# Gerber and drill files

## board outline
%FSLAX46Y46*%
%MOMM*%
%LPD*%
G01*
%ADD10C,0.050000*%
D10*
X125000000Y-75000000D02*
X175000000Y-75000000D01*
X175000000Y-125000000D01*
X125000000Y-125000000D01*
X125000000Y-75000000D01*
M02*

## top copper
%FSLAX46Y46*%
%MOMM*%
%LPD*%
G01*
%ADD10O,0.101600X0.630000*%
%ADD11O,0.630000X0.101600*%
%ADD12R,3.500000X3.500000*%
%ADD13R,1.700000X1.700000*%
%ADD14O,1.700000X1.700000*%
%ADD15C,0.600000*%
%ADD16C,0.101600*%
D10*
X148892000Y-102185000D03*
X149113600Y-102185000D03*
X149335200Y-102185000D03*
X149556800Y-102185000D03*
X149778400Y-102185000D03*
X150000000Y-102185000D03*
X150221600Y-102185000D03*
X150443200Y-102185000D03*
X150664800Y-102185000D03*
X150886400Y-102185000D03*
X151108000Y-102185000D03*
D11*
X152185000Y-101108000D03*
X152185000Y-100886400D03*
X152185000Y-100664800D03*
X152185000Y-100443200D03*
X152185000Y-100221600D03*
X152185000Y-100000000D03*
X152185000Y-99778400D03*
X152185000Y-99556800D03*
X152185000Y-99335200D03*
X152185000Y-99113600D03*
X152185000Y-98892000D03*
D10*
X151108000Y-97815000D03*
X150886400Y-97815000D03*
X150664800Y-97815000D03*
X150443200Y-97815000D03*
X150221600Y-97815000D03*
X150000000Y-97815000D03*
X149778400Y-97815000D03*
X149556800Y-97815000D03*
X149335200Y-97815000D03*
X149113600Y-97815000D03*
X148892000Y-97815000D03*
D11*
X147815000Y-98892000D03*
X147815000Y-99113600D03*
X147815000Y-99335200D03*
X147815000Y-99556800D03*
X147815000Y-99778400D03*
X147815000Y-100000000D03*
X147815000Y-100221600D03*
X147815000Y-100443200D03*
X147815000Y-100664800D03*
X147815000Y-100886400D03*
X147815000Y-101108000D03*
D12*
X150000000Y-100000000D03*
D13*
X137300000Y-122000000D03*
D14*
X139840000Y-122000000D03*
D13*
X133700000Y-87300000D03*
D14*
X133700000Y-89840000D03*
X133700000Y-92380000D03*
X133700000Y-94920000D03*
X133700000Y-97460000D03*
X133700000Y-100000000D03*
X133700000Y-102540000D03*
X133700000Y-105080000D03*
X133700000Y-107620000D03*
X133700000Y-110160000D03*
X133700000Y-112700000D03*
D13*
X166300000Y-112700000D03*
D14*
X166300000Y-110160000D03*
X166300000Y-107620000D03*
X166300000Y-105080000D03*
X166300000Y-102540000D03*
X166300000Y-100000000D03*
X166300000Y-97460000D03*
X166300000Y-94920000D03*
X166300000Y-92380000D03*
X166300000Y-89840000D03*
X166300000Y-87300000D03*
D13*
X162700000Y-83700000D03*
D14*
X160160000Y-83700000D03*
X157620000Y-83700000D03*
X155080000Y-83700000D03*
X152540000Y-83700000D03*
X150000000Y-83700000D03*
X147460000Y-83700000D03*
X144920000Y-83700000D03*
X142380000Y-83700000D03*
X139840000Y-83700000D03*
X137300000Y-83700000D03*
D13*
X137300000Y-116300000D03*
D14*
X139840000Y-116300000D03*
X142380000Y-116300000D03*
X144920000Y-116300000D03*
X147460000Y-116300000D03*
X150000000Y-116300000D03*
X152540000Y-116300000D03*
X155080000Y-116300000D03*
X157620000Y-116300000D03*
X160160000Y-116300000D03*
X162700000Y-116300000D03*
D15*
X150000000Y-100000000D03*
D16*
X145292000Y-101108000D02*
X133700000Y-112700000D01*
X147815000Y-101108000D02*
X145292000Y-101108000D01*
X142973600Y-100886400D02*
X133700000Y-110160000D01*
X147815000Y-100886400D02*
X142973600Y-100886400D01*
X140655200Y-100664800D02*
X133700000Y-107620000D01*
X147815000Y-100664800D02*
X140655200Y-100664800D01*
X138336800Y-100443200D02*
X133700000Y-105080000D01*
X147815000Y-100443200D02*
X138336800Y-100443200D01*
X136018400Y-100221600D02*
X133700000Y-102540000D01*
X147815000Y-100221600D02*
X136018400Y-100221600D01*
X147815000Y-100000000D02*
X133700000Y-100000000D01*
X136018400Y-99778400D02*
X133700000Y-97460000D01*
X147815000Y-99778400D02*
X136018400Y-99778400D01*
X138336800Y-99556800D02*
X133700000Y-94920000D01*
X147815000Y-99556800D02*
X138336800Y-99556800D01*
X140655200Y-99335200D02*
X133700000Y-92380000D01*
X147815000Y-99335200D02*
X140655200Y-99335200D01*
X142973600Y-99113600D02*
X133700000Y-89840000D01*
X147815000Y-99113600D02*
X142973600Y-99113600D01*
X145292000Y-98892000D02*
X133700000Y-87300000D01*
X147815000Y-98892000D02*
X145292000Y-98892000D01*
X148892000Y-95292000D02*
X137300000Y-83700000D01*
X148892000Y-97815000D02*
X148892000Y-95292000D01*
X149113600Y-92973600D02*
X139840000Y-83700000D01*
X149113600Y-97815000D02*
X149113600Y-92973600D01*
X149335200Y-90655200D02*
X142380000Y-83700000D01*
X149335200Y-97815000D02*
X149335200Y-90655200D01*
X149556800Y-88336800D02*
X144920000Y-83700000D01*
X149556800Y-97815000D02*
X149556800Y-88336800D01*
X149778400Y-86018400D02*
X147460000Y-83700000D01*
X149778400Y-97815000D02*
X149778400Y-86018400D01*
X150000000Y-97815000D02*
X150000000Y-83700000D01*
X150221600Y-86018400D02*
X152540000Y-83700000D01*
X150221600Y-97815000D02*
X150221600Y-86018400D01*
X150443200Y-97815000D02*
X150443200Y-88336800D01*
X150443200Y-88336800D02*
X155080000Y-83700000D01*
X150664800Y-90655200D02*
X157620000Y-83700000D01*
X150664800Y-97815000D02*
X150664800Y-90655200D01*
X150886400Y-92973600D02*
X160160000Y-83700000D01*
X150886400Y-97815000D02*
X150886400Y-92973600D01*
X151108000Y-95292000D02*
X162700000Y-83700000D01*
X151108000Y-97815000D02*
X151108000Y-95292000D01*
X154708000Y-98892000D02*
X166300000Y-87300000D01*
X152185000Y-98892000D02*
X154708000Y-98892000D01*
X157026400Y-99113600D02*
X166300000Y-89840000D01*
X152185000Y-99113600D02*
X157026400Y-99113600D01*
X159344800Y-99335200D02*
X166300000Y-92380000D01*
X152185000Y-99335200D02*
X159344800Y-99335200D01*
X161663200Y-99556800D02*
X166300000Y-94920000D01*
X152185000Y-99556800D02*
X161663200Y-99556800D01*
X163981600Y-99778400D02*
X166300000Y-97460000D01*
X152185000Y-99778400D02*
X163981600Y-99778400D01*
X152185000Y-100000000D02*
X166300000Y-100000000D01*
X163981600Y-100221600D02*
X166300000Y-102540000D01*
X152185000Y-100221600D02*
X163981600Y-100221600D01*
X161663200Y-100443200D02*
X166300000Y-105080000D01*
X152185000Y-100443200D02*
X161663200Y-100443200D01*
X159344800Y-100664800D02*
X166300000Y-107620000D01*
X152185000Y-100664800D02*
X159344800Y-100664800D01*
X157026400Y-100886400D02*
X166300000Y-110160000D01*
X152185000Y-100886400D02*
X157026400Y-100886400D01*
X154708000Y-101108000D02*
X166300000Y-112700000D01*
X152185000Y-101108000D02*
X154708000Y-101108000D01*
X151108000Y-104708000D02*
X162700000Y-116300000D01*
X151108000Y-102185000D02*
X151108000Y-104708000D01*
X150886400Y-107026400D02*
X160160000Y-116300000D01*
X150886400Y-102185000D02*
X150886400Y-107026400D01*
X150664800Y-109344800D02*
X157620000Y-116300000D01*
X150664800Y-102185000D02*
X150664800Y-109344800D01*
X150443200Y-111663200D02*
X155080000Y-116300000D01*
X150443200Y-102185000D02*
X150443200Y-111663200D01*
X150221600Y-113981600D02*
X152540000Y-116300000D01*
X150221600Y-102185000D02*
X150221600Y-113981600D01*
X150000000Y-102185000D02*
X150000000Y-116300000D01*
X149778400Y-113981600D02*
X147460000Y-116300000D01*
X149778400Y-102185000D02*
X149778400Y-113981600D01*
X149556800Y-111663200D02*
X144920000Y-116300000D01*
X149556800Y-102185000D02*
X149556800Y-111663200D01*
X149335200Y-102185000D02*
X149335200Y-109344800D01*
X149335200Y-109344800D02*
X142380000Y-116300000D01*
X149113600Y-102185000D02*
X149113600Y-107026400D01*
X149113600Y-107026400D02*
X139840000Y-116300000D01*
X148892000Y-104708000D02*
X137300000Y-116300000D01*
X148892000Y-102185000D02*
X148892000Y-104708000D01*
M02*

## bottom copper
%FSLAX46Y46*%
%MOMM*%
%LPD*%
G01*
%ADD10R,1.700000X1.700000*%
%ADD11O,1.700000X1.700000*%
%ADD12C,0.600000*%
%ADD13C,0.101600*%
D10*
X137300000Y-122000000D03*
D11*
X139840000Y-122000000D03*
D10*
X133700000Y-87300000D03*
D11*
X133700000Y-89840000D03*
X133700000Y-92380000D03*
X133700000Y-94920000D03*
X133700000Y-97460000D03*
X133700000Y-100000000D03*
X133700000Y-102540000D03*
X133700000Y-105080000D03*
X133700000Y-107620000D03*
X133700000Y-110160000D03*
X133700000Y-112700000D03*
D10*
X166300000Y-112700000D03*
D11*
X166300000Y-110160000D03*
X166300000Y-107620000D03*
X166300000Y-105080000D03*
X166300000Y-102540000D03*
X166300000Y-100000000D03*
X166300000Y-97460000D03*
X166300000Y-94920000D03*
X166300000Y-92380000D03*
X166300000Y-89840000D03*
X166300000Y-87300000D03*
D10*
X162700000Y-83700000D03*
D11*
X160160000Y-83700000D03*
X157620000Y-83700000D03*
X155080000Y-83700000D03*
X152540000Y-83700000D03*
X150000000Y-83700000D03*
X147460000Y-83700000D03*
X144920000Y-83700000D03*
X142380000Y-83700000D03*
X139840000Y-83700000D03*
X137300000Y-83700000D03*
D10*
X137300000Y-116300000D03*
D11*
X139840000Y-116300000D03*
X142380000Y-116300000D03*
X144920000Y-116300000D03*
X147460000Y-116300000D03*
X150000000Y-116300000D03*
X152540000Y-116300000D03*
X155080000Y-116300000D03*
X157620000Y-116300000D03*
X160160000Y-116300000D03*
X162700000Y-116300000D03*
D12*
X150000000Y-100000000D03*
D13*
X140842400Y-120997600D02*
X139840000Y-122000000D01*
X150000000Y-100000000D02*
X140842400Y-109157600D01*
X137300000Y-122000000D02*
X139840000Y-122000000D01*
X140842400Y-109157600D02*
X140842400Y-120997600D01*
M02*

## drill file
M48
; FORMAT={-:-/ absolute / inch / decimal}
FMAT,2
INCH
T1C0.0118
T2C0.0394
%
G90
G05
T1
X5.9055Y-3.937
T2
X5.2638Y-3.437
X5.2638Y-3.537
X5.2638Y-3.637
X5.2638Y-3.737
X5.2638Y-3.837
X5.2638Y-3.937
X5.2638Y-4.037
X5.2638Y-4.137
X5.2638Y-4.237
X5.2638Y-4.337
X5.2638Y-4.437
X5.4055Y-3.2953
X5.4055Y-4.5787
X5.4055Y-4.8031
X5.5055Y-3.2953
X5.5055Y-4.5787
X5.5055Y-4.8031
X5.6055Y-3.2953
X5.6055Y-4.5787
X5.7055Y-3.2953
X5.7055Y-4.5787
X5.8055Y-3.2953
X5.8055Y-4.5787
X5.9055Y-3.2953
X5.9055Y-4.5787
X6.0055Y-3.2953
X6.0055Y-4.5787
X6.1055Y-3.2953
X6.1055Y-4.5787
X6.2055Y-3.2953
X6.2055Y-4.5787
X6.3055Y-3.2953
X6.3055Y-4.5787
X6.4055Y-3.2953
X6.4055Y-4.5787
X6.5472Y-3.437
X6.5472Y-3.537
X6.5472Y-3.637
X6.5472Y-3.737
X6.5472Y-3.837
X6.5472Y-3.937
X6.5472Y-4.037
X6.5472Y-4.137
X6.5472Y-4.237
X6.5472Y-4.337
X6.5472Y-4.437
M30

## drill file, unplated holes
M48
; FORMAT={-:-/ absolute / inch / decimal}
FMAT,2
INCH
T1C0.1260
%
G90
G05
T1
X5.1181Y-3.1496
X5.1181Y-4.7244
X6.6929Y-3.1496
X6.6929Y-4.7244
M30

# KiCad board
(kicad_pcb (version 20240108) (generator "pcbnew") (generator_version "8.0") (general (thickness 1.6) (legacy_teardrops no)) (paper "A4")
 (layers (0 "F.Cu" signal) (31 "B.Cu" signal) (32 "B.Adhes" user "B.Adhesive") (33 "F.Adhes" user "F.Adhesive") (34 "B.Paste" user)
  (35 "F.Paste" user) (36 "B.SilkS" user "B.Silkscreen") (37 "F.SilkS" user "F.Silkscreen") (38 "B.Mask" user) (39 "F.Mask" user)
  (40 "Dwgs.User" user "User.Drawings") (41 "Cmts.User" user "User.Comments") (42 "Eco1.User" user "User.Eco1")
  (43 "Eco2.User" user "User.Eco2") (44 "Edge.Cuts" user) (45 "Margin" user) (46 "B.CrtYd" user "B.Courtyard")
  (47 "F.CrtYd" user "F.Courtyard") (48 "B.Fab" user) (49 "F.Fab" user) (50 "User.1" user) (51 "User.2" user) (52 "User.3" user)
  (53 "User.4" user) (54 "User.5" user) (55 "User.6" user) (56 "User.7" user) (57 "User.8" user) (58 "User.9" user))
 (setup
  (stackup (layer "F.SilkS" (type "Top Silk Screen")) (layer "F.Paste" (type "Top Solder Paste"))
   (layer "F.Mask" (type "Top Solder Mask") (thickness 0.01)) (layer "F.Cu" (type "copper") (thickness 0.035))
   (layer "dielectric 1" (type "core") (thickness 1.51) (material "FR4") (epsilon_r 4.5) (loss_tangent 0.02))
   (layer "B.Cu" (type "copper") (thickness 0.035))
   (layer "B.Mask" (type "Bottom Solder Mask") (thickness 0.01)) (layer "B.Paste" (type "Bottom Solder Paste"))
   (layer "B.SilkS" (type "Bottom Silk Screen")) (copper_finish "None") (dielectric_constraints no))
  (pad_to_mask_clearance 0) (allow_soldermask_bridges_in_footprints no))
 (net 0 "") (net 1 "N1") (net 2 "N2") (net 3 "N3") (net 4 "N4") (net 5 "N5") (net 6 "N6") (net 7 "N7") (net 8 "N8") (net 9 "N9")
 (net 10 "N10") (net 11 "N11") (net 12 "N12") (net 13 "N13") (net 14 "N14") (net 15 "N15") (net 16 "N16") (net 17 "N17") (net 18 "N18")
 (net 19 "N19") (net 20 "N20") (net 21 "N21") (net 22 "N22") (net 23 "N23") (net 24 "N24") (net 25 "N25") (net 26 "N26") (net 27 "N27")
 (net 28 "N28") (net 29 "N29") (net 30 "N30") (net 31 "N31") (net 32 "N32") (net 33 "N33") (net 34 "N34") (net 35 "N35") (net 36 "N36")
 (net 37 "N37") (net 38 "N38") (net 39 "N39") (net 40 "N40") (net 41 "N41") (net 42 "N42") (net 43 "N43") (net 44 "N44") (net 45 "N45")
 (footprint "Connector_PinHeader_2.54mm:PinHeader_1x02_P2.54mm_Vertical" (layer "F.Cu") (at 137.3 122 90)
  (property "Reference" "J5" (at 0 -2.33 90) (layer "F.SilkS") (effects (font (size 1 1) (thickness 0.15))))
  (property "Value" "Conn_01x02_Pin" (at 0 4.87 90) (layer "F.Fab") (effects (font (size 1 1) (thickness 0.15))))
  (pad "1" thru_hole rect (at 0 0 90) (size 1.7 1.7) (drill 1) (layers "*.Cu" "*.Mask") (remove_unused_layers no) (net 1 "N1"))
  (pad "2" thru_hole oval (at 0 2.54 90) (size 1.7 1.7) (drill 1) (layers "*.Cu" "*.Mask") (remove_unused_layers no) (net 1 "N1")))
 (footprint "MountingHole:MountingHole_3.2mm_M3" (layer "F.Cu") (at 130 120)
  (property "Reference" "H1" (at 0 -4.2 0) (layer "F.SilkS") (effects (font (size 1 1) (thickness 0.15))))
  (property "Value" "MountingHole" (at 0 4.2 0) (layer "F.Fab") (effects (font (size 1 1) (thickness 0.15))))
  (pad "" np_thru_hole circle (at 0 0) (size 3.2 3.2) (drill 3.2) (layers "*.Cu" "*.Mask")))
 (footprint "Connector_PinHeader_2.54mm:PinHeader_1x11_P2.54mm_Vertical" (layer "F.Cu") (at 133.7 87.3)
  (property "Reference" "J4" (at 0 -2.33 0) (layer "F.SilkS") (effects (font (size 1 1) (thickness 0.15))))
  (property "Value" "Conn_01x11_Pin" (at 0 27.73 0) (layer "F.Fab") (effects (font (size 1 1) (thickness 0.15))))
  (pad "1" thru_hole rect (at 0 0) (size 1.7 1.7) (drill 1) (layers "*.Cu" "*.Mask") (remove_unused_layers no) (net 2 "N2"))
  (pad "2" thru_hole oval (at 0 2.54) (size 1.7 1.7) (drill 1) (layers "*.Cu" "*.Mask") (remove_unused_layers no) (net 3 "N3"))
  (pad "3" thru_hole oval (at 0 5.08) (size 1.7 1.7) (drill 1) (layers "*.Cu" "*.Mask") (remove_unused_layers no) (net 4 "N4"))
  (pad "4" thru_hole oval (at 0 7.62) (size 1.7 1.7) (drill 1) (layers "*.Cu" "*.Mask") (remove_unused_layers no) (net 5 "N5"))
  (pad "5" thru_hole oval (at 0 10.16) (size 1.7 1.7) (drill 1) (layers "*.Cu" "*.Mask") (remove_unused_layers no) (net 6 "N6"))
  (pad "6" thru_hole oval (at 0 12.7) (size 1.7 1.7) (drill 1) (layers "*.Cu" "*.Mask") (remove_unused_layers no) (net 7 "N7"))
  (pad "7" thru_hole oval (at 0 15.24) (size 1.7 1.7) (drill 1) (layers "*.Cu" "*.Mask") (remove_unused_layers no) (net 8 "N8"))
  (pad "8" thru_hole oval (at 0 17.78) (size 1.7 1.7) (drill 1) (layers "*.Cu" "*.Mask") (remove_unused_layers no) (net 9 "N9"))
  (pad "9" thru_hole oval (at 0 20.32) (size 1.7 1.7) (drill 1) (layers "*.Cu" "*.Mask") (remove_unused_layers no) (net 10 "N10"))
  (pad "10" thru_hole oval (at 0 22.86) (size 1.7 1.7) (drill 1) (layers "*.Cu" "*.Mask") (remove_unused_layers no) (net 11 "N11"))
  (pad "11" thru_hole oval (at 0 25.4) (size 1.7 1.7) (drill 1) (layers "*.Cu" "*.Mask") (remove_unused_layers no) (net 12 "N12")))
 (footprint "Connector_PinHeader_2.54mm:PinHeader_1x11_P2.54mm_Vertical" (layer "F.Cu") (at 166.3 112.7 180)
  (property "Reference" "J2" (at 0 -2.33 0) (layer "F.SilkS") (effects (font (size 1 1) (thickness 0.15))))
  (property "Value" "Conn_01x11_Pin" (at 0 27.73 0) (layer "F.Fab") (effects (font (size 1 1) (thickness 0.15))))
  (pad "1" thru_hole rect (at 0 0 180) (size 1.7 1.7) (drill 1) (layers "*.Cu" "*.Mask") (remove_unused_layers no) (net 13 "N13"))
  (pad "2" thru_hole oval (at 0 2.54 180) (size 1.7 1.7) (drill 1) (layers "*.Cu" "*.Mask") (remove_unused_layers no) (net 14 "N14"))
  (pad "3" thru_hole oval (at 0 5.08 180) (size 1.7 1.7) (drill 1) (layers "*.Cu" "*.Mask") (remove_unused_layers no) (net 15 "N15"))
  (pad "4" thru_hole oval (at 0 7.62 180) (size 1.7 1.7) (drill 1) (layers "*.Cu" "*.Mask") (remove_unused_layers no) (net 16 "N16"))
  (pad "5" thru_hole oval (at 0 10.16 180) (size 1.7 1.7) (drill 1) (layers "*.Cu" "*.Mask") (remove_unused_layers no) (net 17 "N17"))
  (pad "6" thru_hole oval (at 0 12.7 180) (size 1.7 1.7) (drill 1) (layers "*.Cu" "*.Mask") (remove_unused_layers no) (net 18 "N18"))
  (pad "7" thru_hole oval (at 0 15.24 180) (size 1.7 1.7) (drill 1) (layers "*.Cu" "*.Mask") (remove_unused_layers no) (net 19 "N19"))
  (pad "8" thru_hole oval (at 0 17.78 180) (size 1.7 1.7) (drill 1) (layers "*.Cu" "*.Mask") (remove_unused_layers no) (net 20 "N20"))
  (pad "9" thru_hole oval (at 0 20.32 180) (size 1.7 1.7) (drill 1) (layers "*.Cu" "*.Mask") (remove_unused_layers no) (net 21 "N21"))
  (pad "10" thru_hole oval (at 0 22.86 180) (size 1.7 1.7) (drill 1) (layers "*.Cu" "*.Mask") (remove_unused_layers no) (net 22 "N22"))
  (pad "11" thru_hole oval (at 0 25.4 180) (size 1.7 1.7) (drill 1) (layers "*.Cu" "*.Mask") (remove_unused_layers no) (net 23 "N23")))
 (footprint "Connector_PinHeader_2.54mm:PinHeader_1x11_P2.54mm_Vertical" (layer "F.Cu") (at 162.7 83.7 -90)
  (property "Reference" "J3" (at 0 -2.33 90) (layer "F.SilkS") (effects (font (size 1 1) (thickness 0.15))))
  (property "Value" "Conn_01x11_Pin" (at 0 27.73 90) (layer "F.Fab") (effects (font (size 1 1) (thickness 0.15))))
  (pad "1" thru_hole rect (at 0 0 270) (size 1.7 1.7) (drill 1) (layers "*.Cu" "*.Mask") (remove_unused_layers no) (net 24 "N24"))
  (pad "2" thru_hole oval (at 0 2.54 270) (size 1.7 1.7) (drill 1) (layers "*.Cu" "*.Mask") (remove_unused_layers no) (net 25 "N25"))
  (pad "3" thru_hole oval (at 0 5.08 270) (size 1.7 1.7) (drill 1) (layers "*.Cu" "*.Mask") (remove_unused_layers no) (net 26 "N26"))
  (pad "4" thru_hole oval (at 0 7.62 270) (size 1.7 1.7) (drill 1) (layers "*.Cu" "*.Mask") (remove_unused_layers no) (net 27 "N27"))
  (pad "5" thru_hole oval (at 0 10.16 270) (size 1.7 1.7) (drill 1) (layers "*.Cu" "*.Mask") (remove_unused_layers no) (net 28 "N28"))
  (pad "6" thru_hole oval (at 0 12.7 270) (size 1.7 1.7) (drill 1) (layers "*.Cu" "*.Mask") (remove_unused_layers no) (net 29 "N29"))
  (pad "7" thru_hole oval (at 0 15.24 270) (size 1.7 1.7) (drill 1) (layers "*.Cu" "*.Mask") (remove_unused_layers no) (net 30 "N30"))
  (pad "8" thru_hole oval (at 0 17.78 270) (size 1.7 1.7) (drill 1) (layers "*.Cu" "*.Mask") (remove_unused_layers no) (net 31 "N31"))
  (pad "9" thru_hole oval (at 0 20.32 270) (size 1.7 1.7) (drill 1) (layers "*.Cu" "*.Mask") (remove_unused_layers no) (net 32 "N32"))
  (pad "10" thru_hole oval (at 0 22.86 270) (size 1.7 1.7) (drill 1) (layers "*.Cu" "*.Mask") (remove_unused_layers no) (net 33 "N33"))
  (pad "11" thru_hole oval (at 0 25.4 270) (size 1.7 1.7) (drill 1) (layers "*.Cu" "*.Mask") (remove_unused_layers no) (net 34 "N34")))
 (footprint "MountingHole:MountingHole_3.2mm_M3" (layer "F.Cu") (at 170 120)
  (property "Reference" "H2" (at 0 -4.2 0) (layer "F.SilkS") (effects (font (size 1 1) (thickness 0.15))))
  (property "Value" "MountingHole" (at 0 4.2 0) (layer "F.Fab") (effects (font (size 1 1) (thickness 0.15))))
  (pad "" np_thru_hole circle (at 0 0) (size 3.2 3.2) (drill 3.2) (layers "*.Cu" "*.Mask")))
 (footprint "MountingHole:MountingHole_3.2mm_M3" (layer "F.Cu") (at 170 80)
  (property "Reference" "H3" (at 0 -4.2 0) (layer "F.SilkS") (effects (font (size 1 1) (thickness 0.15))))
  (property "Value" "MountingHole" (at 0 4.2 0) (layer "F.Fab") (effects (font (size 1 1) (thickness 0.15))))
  (pad "" np_thru_hole circle (at 0 0) (size 3.2 3.2) (drill 3.2) (layers "*.Cu" "*.Mask")))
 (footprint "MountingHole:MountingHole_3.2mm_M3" (layer "F.Cu") (at 130 80)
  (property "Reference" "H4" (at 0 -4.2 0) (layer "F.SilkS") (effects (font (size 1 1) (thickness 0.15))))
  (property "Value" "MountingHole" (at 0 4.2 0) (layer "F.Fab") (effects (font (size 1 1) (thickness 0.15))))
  (pad "" np_thru_hole circle (at 0 0) (size 3.2 3.2) (drill 3.2) (layers "*.Cu" "*.Mask")))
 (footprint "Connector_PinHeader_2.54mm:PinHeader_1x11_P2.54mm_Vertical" (layer "F.Cu") (at 137.3 116.3 90)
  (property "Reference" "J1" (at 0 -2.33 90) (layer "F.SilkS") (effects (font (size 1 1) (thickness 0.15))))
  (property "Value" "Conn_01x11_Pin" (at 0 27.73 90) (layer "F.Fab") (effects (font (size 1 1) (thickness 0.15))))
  (pad "1" thru_hole rect (at 0 0 90) (size 1.7 1.7) (drill 1) (layers "*.Cu" "*.Mask") (remove_unused_layers no) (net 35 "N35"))
  (pad "2" thru_hole oval (at 0 2.54 90) (size 1.7 1.7) (drill 1) (layers "*.Cu" "*.Mask") (remove_unused_layers no) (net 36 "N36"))
  (pad "3" thru_hole oval (at 0 5.08 90) (size 1.7 1.7) (drill 1) (layers "*.Cu" "*.Mask") (remove_unused_layers no) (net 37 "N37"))
  (pad "4" thru_hole oval (at 0 7.62 90) (size 1.7 1.7) (drill 1) (layers "*.Cu" "*.Mask") (remove_unused_layers no) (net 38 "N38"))
  (pad "5" thru_hole oval (at 0 10.16 90) (size 1.7 1.7) (drill 1) (layers "*.Cu" "*.Mask") (remove_unused_layers no) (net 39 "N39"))
  (pad "6" thru_hole oval (at 0 12.7 90) (size 1.7 1.7) (drill 1) (layers "*.Cu" "*.Mask") (remove_unused_layers no) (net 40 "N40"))
  (pad "7" thru_hole oval (at 0 15.24 90) (size 1.7 1.7) (drill 1) (layers "*.Cu" "*.Mask") (remove_unused_layers no) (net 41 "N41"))
  (pad "8" thru_hole oval (at 0 17.78 90) (size 1.7 1.7) (drill 1) (layers "*.Cu" "*.Mask") (remove_unused_layers no) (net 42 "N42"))
  (pad "9" thru_hole oval (at 0 20.32 90) (size 1.7 1.7) (drill 1) (layers "*.Cu" "*.Mask") (remove_unused_layers no) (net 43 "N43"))
  (pad "10" thru_hole oval (at 0 22.86 90) (size 1.7 1.7) (drill 1) (layers "*.Cu" "*.Mask") (remove_unused_layers no) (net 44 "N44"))
  (pad "11" thru_hole oval (at 0 25.4 90) (size 1.7 1.7) (drill 1) (layers "*.Cu" "*.Mask") (remove_unused_layers no) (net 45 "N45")))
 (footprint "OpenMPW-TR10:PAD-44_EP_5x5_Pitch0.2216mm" (layer "F.Cu") (at 150 100 90)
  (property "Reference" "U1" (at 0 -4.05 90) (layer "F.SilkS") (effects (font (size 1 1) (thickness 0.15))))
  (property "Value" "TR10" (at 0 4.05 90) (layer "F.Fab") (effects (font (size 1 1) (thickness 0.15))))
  (pad "" smd rect (at -1.3125 -1.3125 90) (size 0.875 0.875) (layers "F.Paste") (thermal_bridge_angle 45))
  (pad "" smd rect (at -1.3125 -0.4375 90) (size 0.875 0.875) (layers "F.Paste") (thermal_bridge_angle 45))
  (pad "" smd rect (at -1.3125 0.4375 90) (size 0.875 0.875) (layers "F.Paste") (thermal_bridge_angle 45))
  (pad "" smd rect (at -1.3125 1.3125 90) (size 0.875 0.875) (layers "F.Paste") (thermal_bridge_angle 45))
  (pad "" smd rect (at -0.4375 -1.3125 90) (size 0.875 0.875) (layers "F.Paste") (thermal_bridge_angle 45))
  (pad "" smd rect (at -0.4375 -0.4375 90) (size 0.875 0.875) (layers "F.Paste") (thermal_bridge_angle 45))
  (pad "" smd rect (at -0.4375 0.4375 90) (size 0.875 0.875) (layers "F.Paste") (thermal_bridge_angle 45))
  (pad "" smd rect (at -0.4375 1.3125 90) (size 0.875 0.875) (layers "F.Paste") (thermal_bridge_angle 45))
  (pad "" smd rect (at 0.4375 -1.3125 90) (size 0.875 0.875) (layers "F.Paste") (thermal_bridge_angle 45))
  (pad "" smd rect (at 0.4375 -0.4375 90) (size 0.875 0.875) (layers "F.Paste") (thermal_bridge_angle 45))
  (pad "" smd rect (at 0.4375 0.4375 90) (size 0.875 0.875) (layers "F.Paste") (thermal_bridge_angle 45))
  (pad "" smd rect (at 0.4375 1.3125 90) (size 0.875 0.875) (layers "F.Paste") (thermal_bridge_angle 45))
  (pad "" smd rect (at 1.3125 -1.3125 90) (size 0.875 0.875) (layers "F.Paste") (thermal_bridge_angle 45))
  (pad "" smd rect (at 1.3125 -0.4375 90) (size 0.875 0.875) (layers "F.Paste") (thermal_bridge_angle 45))
  (pad "" smd rect (at 1.3125 0.4375 90) (size 0.875 0.875) (layers "F.Paste") (thermal_bridge_angle 45))
  (pad "" smd rect (at 1.3125 1.3125 90) (size 0.875 0.875) (layers "F.Paste") (thermal_bridge_angle 45))
  (pad "1" smd oval (at -2.185 -1.108 180) (size 0.1016 0.63) (layers "F.Cu" "F.Paste" "F.Mask") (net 35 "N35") (thermal_bridge_angle 45))
  (pad "2" smd oval (at -2.185 -0.8864 180) (size 0.1016 0.63) (layers "F.Cu" "F.Paste" "F.Mask") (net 36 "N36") (thermal_bridge_angle 45))
  (pad "3" smd oval (at -2.185 -0.6648 180) (size 0.1016 0.63) (layers "F.Cu" "F.Paste" "F.Mask") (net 37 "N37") (thermal_bridge_angle 45))
  (pad "4" smd oval (at -2.185 -0.4432 180) (size 0.1016 0.63) (layers "F.Cu" "F.Paste" "F.Mask") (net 38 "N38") (thermal_bridge_angle 45))
  (pad "5" smd oval (at -2.185 -0.2216 180) (size 0.1016 0.63) (layers "F.Cu" "F.Paste" "F.Mask") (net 39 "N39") (thermal_bridge_angle 45))
  (pad "6" smd oval (at -2.185 0 180) (size 0.1016 0.63) (layers "F.Cu" "F.Paste" "F.Mask") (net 40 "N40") (thermal_bridge_angle 45))
  (pad "7" smd oval (at -2.185 0.2216 180) (size 0.1016 0.63) (layers "F.Cu" "F.Paste" "F.Mask") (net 41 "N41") (thermal_bridge_angle 45))
  (pad "8" smd oval (at -2.185 0.4432 180) (size 0.1016 0.63) (layers "F.Cu" "F.Paste" "F.Mask") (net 42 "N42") (thermal_bridge_angle 45))
  (pad "9" smd oval (at -2.185 0.6648 180) (size 0.1016 0.63) (layers "F.Cu" "F.Paste" "F.Mask") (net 43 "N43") (thermal_bridge_angle 45))
  (pad "10" smd oval (at -2.185 0.8864 180) (size 0.1016 0.63) (layers "F.Cu" "F.Paste" "F.Mask") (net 44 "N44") (thermal_bridge_angle 45))
  (pad "11" smd oval (at -2.185 1.108 180) (size 0.1016 0.63) (layers "F.Cu" "F.Paste" "F.Mask") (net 45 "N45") (thermal_bridge_angle 45))
  (pad "12" smd oval (at -1.108 2.185 90) (size 0.1016 0.63) (layers "F.Cu" "F.Paste" "F.Mask") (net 13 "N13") (thermal_bridge_angle 45))
  (pad "13" smd oval (at -0.8864 2.185 90) (size 0.1016 0.63) (layers "F.Cu" "F.Paste" "F.Mask") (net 14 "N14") (thermal_bridge_angle 45))
  (pad "14" smd oval (at -0.6648 2.185 90) (size 0.1016 0.63) (layers "F.Cu" "F.Paste" "F.Mask") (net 15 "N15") (thermal_bridge_angle 45))
  (pad "15" smd oval (at -0.4432 2.185 90) (size 0.1016 0.63) (layers "F.Cu" "F.Paste" "F.Mask") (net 16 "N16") (thermal_bridge_angle 45))
  (pad "16" smd oval (at -0.2216 2.185 90) (size 0.1016 0.63) (layers "F.Cu" "F.Paste" "F.Mask") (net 17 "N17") (thermal_bridge_angle 45))
  (pad "17" smd oval (at 0 2.185 90) (size 0.1016 0.63) (layers "F.Cu" "F.Paste" "F.Mask") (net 18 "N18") (thermal_bridge_angle 45))
  (pad "18" smd oval (at 0.2216 2.185 90) (size 0.1016 0.63) (layers "F.Cu" "F.Paste" "F.Mask") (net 19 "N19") (thermal_bridge_angle 45))
  (pad "19" smd oval (at 0.4432 2.185 90) (size 0.1016 0.63) (layers "F.Cu" "F.Paste" "F.Mask") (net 20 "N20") (thermal_bridge_angle 45))
  (pad "20" smd oval (at 0.6648 2.185 90) (size 0.1016 0.63) (layers "F.Cu" "F.Paste" "F.Mask") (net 21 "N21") (thermal_bridge_angle 45))
  (pad "21" smd oval (at 0.8864 2.185 90) (size 0.1016 0.63) (layers "F.Cu" "F.Paste" "F.Mask") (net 22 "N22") (thermal_bridge_angle 45))
  (pad "22" smd oval (at 1.108 2.185 90) (size 0.1016 0.63) (layers "F.Cu" "F.Paste" "F.Mask") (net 23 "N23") (thermal_bridge_angle 45))
  (pad "23" smd oval (at 2.185 1.108 180) (size 0.1016 0.63) (layers "F.Cu" "F.Paste" "F.Mask") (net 24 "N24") (thermal_bridge_angle 45))
  (pad "24" smd oval (at 2.185 0.8864 180) (size 0.1016 0.63) (layers "F.Cu" "F.Paste" "F.Mask") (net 25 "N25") (thermal_bridge_angle 45))
  (pad "25" smd oval (at 2.185 0.6648 180) (size 0.1016 0.63) (layers "F.Cu" "F.Paste" "F.Mask") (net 26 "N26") (thermal_bridge_angle 45))
  (pad "26" smd oval (at 2.185 0.4432 180) (size 0.1016 0.63) (layers "F.Cu" "F.Paste" "F.Mask") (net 27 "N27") (thermal_bridge_angle 45))
  (pad "27" smd oval (at 2.185 0.2216 180) (size 0.1016 0.63) (layers "F.Cu" "F.Paste" "F.Mask") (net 28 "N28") (thermal_bridge_angle 45))
  (pad "28" smd oval (at 2.185 0 180) (size 0.1016 0.63) (layers "F.Cu" "F.Paste" "F.Mask") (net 29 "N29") (thermal_bridge_angle 45))
  (pad "29" smd oval (at 2.185 -0.2216 180) (size 0.1016 0.63) (layers "F.Cu" "F.Paste" "F.Mask") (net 30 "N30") (thermal_bridge_angle 45))
  (pad "30" smd oval (at 2.185 -0.4432 180) (size 0.1016 0.63) (layers "F.Cu" "F.Paste" "F.Mask") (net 31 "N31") (thermal_bridge_angle 45))
  (pad "31" smd oval (at 2.185 -0.6648 180) (size 0.1016 0.63) (layers "F.Cu" "F.Paste" "F.Mask") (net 32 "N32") (thermal_bridge_angle 45))
  (pad "32" smd oval (at 2.185 -0.8864 180) (size 0.1016 0.63) (layers "F.Cu" "F.Paste" "F.Mask") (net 33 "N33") (thermal_bridge_angle 45))
  (pad "33" smd oval (at 2.185 -1.108 180) (size 0.1016 0.63) (layers "F.Cu" "F.Paste" "F.Mask") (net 34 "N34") (thermal_bridge_angle 45))
  (pad "34" smd oval (at 1.108 -2.185 90) (size 0.1016 0.63) (layers "F.Cu" "F.Paste" "F.Mask") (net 2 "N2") (thermal_bridge_angle 45))
  (pad "35" smd oval (at 0.8864 -2.185 90) (size 0.1016 0.63) (layers "F.Cu" "F.Paste" "F.Mask") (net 3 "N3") (thermal_bridge_angle 45))
  (pad "36" smd oval (at 0.6648 -2.185 90) (size 0.1016 0.63) (layers "F.Cu" "F.Paste" "F.Mask") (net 4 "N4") (thermal_bridge_angle 45))
  (pad "37" smd oval (at 0.4432 -2.185 90) (size 0.1016 0.63) (layers "F.Cu" "F.Paste" "F.Mask") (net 5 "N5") (thermal_bridge_angle 45))
  (pad "38" smd oval (at 0.2216 -2.185 90) (size 0.1016 0.63) (layers "F.Cu" "F.Paste" "F.Mask") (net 6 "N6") (thermal_bridge_angle 45))
  (pad "39" smd oval (at 0 -2.185 90) (size 0.1016 0.63) (layers "F.Cu" "F.Paste" "F.Mask") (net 7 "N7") (thermal_bridge_angle 45))
  (pad "40" smd oval (at -0.2216 -2.185 90) (size 0.1016 0.63) (layers "F.Cu" "F.Paste" "F.Mask") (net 8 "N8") (thermal_bridge_angle 45))
  (pad "41" smd oval (at -0.4432 -2.185 90) (size 0.1016 0.63) (layers "F.Cu" "F.Paste" "F.Mask") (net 9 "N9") (thermal_bridge_angle 45))
  (pad "42" smd oval (at -0.6648 -2.185 90) (size 0.1016 0.63) (layers "F.Cu" "F.Paste" "F.Mask") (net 10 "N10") (thermal_bridge_angle 45))
  (pad "43" smd oval (at -0.8864 -2.185 90) (size 0.1016 0.63) (layers "F.Cu" "F.Paste" "F.Mask") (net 11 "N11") (thermal_bridge_angle 45))
  (pad "44" smd oval (at -1.108 -2.185 90) (size 0.1016 0.63) (layers "F.Cu" "F.Paste" "F.Mask") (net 12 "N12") (thermal_bridge_angle 45))
  (pad "45" smd rect (at 0 0 90) (size 3.5 3.5) (layers "F.Cu" "F.Mask") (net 1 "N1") (thermal_bridge_angle 45)))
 (gr_rect (start 125 75) (end 175 125) (stroke (width 0.05) (type default)) (fill none) (layer "Edge.Cuts"))
 (segment (start 149.3352 102.185) (end 149.3352 109.3448) (width 0.1016) (layer "F.Cu") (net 37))
 (segment (start 149.3352 109.3448) (end 142.38 116.3) (width 0.1016) (layer "F.Cu") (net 37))
 (segment (start 150.8864 107.0264) (end 160.16 116.3) (width 0.1016) (layer "F.Cu") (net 44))
 (segment (start 150.8864 102.185) (end 150.8864 107.0264) (width 0.1016) (layer "F.Cu") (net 44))
 (segment (start 149.1136 102.185) (end 149.1136 107.0264) (width 0.1016) (layer "F.Cu") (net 36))
 (segment (start 149.1136 107.0264) (end 139.84 116.3) (width 0.1016) (layer "F.Cu") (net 36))
 (segment (start 150.6648 102.185) (end 150.6648 109.3448) (width 0.1016) (layer "F.Cu") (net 43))
 (segment (start 150.6648 109.3448) (end 157.62 116.3) (width 0.1016) (layer "F.Cu") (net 43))
 (segment (start 150.4432 102.185) (end 150.4432 111.6632) (width 0.1016) (layer "F.Cu") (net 42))
 (segment (start 150.4432 111.6632) (end 155.08 116.3) (width 0.1016) (layer "F.Cu") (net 42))
 (segment (start 149.7784 113.9816) (end 147.46 116.3) (width 0.1016) (layer "F.Cu") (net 39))
 (segment (start 149.7784 102.185) (end 149.7784 113.9816) (width 0.1016) (layer "F.Cu") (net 39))
 (segment (start 148.892 104.708) (end 137.3 116.3) (width 0.1016) (layer "F.Cu") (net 35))
 (segment (start 148.892 102.185) (end 148.892 104.708) (width 0.1016) (layer "F.Cu") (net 35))
 (segment (start 151.108 104.708) (end 162.7 116.3) (width 0.1016) (layer "F.Cu") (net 45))
 (segment (start 151.108 102.185) (end 151.108 104.708) (width 0.1016) (layer "F.Cu") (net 45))
 (segment (start 150 102.185) (end 150 116.3) (width 0.1016) (layer "F.Cu") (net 40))
 (segment (start 150.2216 113.9816) (end 152.54 116.3) (width 0.1016) (layer "F.Cu") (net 41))
 (segment (start 150.2216 102.185) (end 150.2216 113.9816) (width 0.1016) (layer "F.Cu") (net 41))
 (segment (start 149.5568 111.6632) (end 144.92 116.3) (width 0.1016) (layer "F.Cu") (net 38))
 (segment (start 149.5568 102.185) (end 149.5568 111.6632) (width 0.1016) (layer "F.Cu") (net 38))
 (segment (start 154.708 98.892) (end 166.3 87.3) (width 0.1016) (layer "F.Cu") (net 23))
 (segment (start 152.185 98.892) (end 154.708 98.892) (width 0.1016) (layer "F.Cu") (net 23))
 (segment (start 154.708 101.108) (end 166.3 112.7) (width 0.1016) (layer "F.Cu") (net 13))
 (segment (start 152.185 101.108) (end 154.708 101.108) (width 0.1016) (layer "F.Cu") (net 13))
 (segment (start 152.185 100.6648) (end 159.3448 100.6648) (width 0.1016) (layer "F.Cu") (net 15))
 (segment (start 159.3448 100.6648) (end 166.3 107.62) (width 0.1016) (layer "F.Cu") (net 15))
 (segment (start 152.185 99.1136) (end 157.0264 99.1136) (width 0.1016) (layer "F.Cu") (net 22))
 (segment (start 157.0264 99.1136) (end 166.3 89.84) (width 0.1016) (layer "F.Cu") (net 22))
 (segment (start 163.9816 99.7784) (end 166.3 97.46) (width 0.1016) (layer "F.Cu") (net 19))
 (segment (start 152.185 99.7784) (end 163.9816 99.7784) (width 0.1016) (layer "F.Cu") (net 19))
 (segment (start 152.185 99.5568) (end 161.6632 99.5568) (width 0.1016) (layer "F.Cu") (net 20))
 (segment (start 161.6632 99.5568) (end 166.3 94.92) (width 0.1016) (layer "F.Cu") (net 20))
 (segment (start 152.185 100) (end 166.3 100) (width 0.1016) (layer "F.Cu") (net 18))
 (segment (start 152.185 100.4432) (end 161.6632 100.4432) (width 0.1016) (layer "F.Cu") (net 16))
 (segment (start 161.6632 100.4432) (end 166.3 105.08) (width 0.1016) (layer "F.Cu") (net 16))
 (segment (start 152.185 100.2216) (end 163.9816 100.2216) (width 0.1016) (layer "F.Cu") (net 17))
 (segment (start 163.9816 100.2216) (end 166.3 102.54) (width 0.1016) (layer "F.Cu") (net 17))
 (segment (start 152.185 100.8864) (end 157.0264 100.8864) (width 0.1016) (layer "F.Cu") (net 14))
 (segment (start 157.0264 100.8864) (end 166.3 110.16) (width 0.1016) (layer "F.Cu") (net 14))
 (segment (start 152.185 99.3352) (end 159.3448 99.3352) (width 0.1016) (layer "F.Cu") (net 21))
 (segment (start 159.3448 99.3352) (end 166.3 92.38) (width 0.1016) (layer "F.Cu") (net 21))
 (segment (start 149.1136 97.815) (end 149.1136 92.9736) (width 0.1016) (layer "F.Cu") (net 33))
 (segment (start 149.1136 92.9736) (end 139.84 83.7) (width 0.1016) (layer "F.Cu") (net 33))
 (segment (start 150.8864 92.9736) (end 160.16 83.7) (width 0.1016) (layer "F.Cu") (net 25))
 (segment (start 150.8864 97.815) (end 150.8864 92.9736) (width 0.1016) (layer "F.Cu") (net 25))
 (segment (start 148.892 95.292) (end 137.3 83.7) (width 0.1016) (layer "F.Cu") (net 34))
 (segment (start 148.892 97.815) (end 148.892 95.292) (width 0.1016) (layer "F.Cu") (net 34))
 (segment (start 150.4432 88.3368) (end 155.08 83.7) (width 0.1016) (layer "F.Cu") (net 27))
 (segment (start 150.4432 97.815) (end 150.4432 88.3368) (width 0.1016) (layer "F.Cu") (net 27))
 (segment (start 149.7784 97.815) (end 149.7784 86.0184) (width 0.1016) (layer "F.Cu") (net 30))
 (segment (start 149.7784 86.0184) (end 147.46 83.7) (width 0.1016) (layer "F.Cu") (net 30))
 (segment (start 149.3352 90.6552) (end 142.38 83.7) (width 0.1016) (layer "F.Cu") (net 32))
 (segment (start 149.3352 97.815) (end 149.3352 90.6552) (width 0.1016) (layer "F.Cu") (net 32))
 (segment (start 150.6648 90.6552) (end 157.62 83.7) (width 0.1016) (layer "F.Cu") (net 26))
 (segment (start 150.6648 97.815) (end 150.6648 90.6552) (width 0.1016) (layer "F.Cu") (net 26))
 (segment (start 150.2216 86.0184) (end 152.54 83.7) (width 0.1016) (layer "F.Cu") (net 28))
 (segment (start 150.2216 97.815) (end 150.2216 86.0184) (width 0.1016) (layer "F.Cu") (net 28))
 (segment (start 151.108 95.292) (end 162.7 83.7) (width 0.1016) (layer "F.Cu") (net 24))
 (segment (start 151.108 97.815) (end 151.108 95.292) (width 0.1016) (layer "F.Cu") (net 24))
 (segment (start 150 97.815) (end 150 83.7) (width 0.1016) (layer "F.Cu") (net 29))
 (segment (start 149.5568 97.815) (end 149.5568 88.3368) (width 0.1016) (layer "F.Cu") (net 31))
 (segment (start 149.5568 88.3368) (end 144.92 83.7) (width 0.1016) (layer "F.Cu") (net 31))
 (segment (start 138.3368 99.5568) (end 133.7 94.92) (width 0.1016) (layer "F.Cu") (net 5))
 (segment (start 147.815 99.5568) (end 138.3368 99.5568) (width 0.1016) (layer "F.Cu") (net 5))
 (segment (start 147.815 99.1136) (end 142.9736 99.1136) (width 0.1016) (layer "F.Cu") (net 3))
 (segment (start 142.9736 99.1136) (end 133.7 89.84) (width 0.1016) (layer "F.Cu") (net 3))
 (segment (start 147.815 100.8864) (end 142.9736 100.8864) (width 0.1016) (layer "F.Cu") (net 11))
 (segment (start 142.9736 100.8864) (end 133.7 110.16) (width 0.1016) (layer "F.Cu") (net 11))
 (segment (start 147.815 100.2216) (end 136.0184 100.2216) (width 0.1016) (layer "F.Cu") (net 8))
 (segment (start 136.0184 100.2216) (end 133.7 102.54) (width 0.1016) (layer "F.Cu") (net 8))
 (segment (start 147.815 100) (end 133.7 100) (width 0.1016) (layer "F.Cu") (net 7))
 (segment (start 140.6552 99.3352) (end 133.7 92.38) (width 0.1016) (layer "F.Cu") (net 4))
 (segment (start 147.815 99.3352) (end 140.6552 99.3352) (width 0.1016) (layer "F.Cu") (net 4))
 (segment (start 147.815 100.4432) (end 138.3368 100.4432) (width 0.1016) (layer "F.Cu") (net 9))
 (segment (start 138.3368 100.4432) (end 133.7 105.08) (width 0.1016) (layer "F.Cu") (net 9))
 (segment (start 145.292 101.108) (end 133.7 112.7) (width 0.1016) (layer "F.Cu") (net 12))
 (segment (start 147.815 101.108) (end 145.292 101.108) (width 0.1016) (layer "F.Cu") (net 12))
 (segment (start 140.6552 100.6648) (end 133.7 107.62) (width 0.1016) (layer "F.Cu") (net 10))
 (segment (start 147.815 100.6648) (end 140.6552 100.6648) (width 0.1016) (layer "F.Cu") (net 10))
 (segment (start 147.815 98.892) (end 145.292 98.892) (width 0.1016) (layer "F.Cu") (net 2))
 (segment (start 145.292 98.892) (end 133.7 87.3) (width 0.1016) (layer "F.Cu") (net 2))
 (segment (start 147.815 99.7784) (end 136.0184 99.7784) (width 0.1016) (layer "F.Cu") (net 6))
 (segment (start 136.0184 99.7784) (end 133.7 97.46) (width 0.1016) (layer "F.Cu") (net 6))
 (via (at 150 100) (size 0.6) (drill 0.3) (layers "F.Cu" "B.Cu") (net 1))
 (segment (start 140.8424 120.9976) (end 139.84 122) (width 0.1016) (layer "B.Cu") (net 1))
 (segment (start 150 100) (end 140.8424 109.1576) (width 0.1016) (layer "B.Cu") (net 1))
 (segment (start 137.3 122) (end 139.84 122) (width 0.1016) (layer "B.Cu") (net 1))
 (segment (start 140.8424 109.1576) (end 140.8424 120.9976) (width 0.1016) (layer "B.Cu") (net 1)))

